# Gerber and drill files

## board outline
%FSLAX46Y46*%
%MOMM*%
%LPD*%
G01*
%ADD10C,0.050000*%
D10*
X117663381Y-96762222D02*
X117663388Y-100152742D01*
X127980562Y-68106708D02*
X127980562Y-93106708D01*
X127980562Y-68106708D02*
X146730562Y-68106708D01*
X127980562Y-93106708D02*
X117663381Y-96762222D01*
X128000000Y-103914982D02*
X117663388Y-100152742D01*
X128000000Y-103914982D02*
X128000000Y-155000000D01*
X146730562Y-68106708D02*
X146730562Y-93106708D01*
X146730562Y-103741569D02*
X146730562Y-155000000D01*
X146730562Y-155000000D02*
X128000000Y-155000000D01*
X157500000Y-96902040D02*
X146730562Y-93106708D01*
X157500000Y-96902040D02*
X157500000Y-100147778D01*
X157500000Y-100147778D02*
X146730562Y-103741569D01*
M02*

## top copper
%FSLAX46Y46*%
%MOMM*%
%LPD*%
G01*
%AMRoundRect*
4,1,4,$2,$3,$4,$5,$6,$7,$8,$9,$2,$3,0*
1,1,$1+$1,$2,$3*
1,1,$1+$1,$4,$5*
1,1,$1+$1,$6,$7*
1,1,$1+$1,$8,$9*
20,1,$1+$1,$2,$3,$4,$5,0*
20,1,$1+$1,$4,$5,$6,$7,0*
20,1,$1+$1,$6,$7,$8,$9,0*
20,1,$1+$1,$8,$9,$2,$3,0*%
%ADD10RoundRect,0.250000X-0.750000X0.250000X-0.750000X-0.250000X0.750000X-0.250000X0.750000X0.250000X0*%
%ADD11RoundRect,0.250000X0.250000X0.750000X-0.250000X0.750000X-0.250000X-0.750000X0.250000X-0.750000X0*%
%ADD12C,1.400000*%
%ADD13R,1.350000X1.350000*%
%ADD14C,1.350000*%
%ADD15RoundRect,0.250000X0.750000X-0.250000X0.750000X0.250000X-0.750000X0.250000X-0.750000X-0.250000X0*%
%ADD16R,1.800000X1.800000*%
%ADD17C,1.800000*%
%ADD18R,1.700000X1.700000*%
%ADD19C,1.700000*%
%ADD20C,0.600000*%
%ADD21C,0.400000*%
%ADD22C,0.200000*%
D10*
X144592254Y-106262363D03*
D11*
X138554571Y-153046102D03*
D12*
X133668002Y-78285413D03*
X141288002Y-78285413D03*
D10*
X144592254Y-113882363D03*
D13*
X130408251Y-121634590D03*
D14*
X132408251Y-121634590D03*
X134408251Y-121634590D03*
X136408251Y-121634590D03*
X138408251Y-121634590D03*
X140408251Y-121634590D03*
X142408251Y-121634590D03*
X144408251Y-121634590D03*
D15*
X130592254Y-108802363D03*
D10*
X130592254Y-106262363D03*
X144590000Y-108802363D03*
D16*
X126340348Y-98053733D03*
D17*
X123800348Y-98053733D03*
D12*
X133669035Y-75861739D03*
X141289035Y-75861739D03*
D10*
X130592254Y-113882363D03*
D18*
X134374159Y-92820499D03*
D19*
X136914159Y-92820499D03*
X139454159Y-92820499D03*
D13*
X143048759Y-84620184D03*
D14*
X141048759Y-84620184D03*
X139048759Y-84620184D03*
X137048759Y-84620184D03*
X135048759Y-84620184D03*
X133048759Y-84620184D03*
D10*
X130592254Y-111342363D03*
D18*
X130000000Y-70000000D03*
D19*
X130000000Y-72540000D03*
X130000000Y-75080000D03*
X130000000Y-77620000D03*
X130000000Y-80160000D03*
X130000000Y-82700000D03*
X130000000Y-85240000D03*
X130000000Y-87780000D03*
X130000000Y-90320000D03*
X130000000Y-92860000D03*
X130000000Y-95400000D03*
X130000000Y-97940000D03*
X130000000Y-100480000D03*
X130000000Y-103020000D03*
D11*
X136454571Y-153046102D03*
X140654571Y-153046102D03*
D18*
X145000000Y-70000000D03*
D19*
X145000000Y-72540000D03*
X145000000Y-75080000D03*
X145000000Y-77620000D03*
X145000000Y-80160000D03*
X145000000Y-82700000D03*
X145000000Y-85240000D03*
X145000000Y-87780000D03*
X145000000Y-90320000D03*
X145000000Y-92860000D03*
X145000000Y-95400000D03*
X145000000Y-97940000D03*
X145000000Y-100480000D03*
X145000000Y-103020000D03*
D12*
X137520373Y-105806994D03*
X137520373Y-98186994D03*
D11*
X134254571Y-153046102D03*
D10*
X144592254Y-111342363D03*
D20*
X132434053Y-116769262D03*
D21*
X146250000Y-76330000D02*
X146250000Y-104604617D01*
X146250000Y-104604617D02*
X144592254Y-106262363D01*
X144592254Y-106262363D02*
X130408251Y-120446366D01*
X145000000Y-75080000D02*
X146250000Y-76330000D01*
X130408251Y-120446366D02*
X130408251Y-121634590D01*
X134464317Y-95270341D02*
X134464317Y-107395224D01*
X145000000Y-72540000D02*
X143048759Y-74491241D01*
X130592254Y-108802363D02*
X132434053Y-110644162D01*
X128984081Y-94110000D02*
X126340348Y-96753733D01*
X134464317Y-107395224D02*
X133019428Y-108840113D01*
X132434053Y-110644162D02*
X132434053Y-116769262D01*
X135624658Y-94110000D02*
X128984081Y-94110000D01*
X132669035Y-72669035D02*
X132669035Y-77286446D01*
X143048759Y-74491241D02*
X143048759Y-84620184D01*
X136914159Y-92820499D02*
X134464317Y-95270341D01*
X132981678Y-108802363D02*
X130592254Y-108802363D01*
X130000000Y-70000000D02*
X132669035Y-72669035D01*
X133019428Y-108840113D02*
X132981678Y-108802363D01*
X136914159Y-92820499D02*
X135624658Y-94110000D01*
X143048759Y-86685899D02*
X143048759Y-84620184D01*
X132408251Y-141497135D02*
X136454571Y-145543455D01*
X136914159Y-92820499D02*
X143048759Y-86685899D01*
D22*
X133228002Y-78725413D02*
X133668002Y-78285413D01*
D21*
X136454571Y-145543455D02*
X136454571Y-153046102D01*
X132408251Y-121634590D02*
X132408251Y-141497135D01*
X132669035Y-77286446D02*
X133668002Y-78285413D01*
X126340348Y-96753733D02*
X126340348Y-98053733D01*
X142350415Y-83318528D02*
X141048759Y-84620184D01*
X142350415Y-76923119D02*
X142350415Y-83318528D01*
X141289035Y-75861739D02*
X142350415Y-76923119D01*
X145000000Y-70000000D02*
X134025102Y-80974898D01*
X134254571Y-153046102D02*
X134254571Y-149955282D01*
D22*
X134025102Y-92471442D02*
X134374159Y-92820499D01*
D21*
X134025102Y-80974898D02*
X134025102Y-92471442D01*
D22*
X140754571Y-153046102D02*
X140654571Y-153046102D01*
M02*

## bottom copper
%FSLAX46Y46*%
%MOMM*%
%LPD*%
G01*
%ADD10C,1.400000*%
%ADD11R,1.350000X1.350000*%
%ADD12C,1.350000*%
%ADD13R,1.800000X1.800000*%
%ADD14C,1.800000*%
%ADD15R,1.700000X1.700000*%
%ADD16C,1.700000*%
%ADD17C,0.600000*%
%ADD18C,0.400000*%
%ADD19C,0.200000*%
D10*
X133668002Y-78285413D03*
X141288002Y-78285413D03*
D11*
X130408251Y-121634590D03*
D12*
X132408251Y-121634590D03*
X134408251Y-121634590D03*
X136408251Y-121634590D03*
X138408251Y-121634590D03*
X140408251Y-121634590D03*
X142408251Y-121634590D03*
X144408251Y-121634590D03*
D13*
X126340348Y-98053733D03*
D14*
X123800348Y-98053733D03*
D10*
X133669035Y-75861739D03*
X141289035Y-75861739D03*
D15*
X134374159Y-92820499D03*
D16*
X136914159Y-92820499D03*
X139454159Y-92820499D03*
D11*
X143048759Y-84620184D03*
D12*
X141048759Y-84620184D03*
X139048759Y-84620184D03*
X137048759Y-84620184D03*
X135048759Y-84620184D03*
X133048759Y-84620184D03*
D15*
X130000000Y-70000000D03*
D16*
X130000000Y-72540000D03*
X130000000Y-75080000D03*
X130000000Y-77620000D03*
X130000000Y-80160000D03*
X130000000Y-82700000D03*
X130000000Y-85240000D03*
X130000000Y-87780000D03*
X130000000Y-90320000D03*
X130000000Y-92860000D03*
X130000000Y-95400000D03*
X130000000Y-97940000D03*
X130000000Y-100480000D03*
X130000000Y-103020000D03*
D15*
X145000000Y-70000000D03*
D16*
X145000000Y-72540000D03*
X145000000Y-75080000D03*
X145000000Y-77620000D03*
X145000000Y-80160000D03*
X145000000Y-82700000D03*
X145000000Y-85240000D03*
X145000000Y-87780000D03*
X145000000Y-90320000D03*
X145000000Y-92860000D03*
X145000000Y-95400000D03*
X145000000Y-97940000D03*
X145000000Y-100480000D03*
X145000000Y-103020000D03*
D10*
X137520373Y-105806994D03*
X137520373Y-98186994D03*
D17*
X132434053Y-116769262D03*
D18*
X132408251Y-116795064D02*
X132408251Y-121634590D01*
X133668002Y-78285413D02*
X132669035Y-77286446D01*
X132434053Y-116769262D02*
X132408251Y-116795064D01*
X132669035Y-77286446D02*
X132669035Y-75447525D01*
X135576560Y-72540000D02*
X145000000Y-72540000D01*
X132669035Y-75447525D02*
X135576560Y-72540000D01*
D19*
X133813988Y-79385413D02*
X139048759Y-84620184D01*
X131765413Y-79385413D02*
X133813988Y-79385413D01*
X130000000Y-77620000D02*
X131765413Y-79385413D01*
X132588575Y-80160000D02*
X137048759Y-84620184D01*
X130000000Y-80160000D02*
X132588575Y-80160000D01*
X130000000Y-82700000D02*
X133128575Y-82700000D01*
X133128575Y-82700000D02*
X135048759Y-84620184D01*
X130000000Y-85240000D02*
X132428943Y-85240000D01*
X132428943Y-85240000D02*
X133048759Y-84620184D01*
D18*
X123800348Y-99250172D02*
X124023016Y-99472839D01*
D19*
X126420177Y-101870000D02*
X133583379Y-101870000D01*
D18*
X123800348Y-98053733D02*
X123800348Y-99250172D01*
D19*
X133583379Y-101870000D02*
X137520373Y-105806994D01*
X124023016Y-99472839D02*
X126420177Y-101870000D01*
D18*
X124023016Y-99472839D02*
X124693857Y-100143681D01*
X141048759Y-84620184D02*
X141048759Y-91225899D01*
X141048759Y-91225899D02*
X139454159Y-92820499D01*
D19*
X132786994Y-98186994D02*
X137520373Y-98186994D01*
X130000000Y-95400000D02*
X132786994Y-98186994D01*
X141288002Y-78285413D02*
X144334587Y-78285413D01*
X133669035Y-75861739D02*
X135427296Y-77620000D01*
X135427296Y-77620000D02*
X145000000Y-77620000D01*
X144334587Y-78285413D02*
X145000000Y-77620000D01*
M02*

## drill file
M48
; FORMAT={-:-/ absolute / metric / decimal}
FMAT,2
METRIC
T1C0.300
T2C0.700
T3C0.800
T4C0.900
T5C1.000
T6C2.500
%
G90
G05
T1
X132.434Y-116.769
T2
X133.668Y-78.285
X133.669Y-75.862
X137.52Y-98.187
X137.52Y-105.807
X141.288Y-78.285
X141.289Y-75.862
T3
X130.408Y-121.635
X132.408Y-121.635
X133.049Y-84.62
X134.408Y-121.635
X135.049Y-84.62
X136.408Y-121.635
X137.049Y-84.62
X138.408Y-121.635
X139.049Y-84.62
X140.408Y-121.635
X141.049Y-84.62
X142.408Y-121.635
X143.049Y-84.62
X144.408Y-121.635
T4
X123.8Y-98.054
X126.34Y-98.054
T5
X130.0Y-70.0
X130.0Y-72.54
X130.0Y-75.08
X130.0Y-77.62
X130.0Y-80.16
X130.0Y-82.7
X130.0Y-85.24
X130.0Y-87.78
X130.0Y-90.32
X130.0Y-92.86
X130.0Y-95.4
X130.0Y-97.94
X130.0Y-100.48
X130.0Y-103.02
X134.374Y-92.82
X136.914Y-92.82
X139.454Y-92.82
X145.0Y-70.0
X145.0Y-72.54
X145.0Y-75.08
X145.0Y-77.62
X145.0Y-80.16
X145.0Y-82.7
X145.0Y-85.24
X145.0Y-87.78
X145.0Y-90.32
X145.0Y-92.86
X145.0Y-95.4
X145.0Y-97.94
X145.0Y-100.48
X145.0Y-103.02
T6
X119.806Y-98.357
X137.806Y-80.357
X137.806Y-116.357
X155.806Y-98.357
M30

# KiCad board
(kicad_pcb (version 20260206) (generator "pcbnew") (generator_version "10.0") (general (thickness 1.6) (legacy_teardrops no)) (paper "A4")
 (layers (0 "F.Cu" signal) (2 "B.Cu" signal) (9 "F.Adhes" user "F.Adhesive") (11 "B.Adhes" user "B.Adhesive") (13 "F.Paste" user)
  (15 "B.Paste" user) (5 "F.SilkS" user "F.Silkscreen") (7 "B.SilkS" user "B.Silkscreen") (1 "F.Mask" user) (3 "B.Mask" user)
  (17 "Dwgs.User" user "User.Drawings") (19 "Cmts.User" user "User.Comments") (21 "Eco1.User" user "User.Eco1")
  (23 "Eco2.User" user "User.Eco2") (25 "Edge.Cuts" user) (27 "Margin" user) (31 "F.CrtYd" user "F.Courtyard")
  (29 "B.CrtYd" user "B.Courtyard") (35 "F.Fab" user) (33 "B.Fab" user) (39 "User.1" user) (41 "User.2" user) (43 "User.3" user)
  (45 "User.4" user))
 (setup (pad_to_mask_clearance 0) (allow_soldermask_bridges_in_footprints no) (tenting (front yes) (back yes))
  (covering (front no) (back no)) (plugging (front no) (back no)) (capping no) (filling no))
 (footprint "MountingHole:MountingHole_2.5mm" (layer "F.Cu") (at 146.772986 83.971093)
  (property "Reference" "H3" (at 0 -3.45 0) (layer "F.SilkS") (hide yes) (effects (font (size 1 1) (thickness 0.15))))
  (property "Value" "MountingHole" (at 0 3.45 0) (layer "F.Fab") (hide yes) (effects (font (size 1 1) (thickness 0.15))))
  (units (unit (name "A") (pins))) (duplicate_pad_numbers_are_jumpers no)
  (pad "" np_thru_hole circle (at 9.033 14.386) (size 2.5 2.5) (drill 2.5) (layers "*.Cu" "*.Mask")))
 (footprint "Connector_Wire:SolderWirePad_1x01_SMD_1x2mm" (layer "F.Cu") (at 144.592254 106.262363 -90)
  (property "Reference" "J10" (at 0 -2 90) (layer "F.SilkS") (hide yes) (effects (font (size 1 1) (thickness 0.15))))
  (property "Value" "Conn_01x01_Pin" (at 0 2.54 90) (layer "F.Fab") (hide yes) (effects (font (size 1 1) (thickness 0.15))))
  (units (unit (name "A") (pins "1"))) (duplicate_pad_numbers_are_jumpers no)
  (pad "1" smd roundrect (at 0 0 270) (size 1 2) (layers "F.Cu" "F.Mask") (roundrect_rratio 0.25) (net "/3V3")))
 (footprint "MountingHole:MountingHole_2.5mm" (layer "F.Cu") (at 118.705986 81.757093)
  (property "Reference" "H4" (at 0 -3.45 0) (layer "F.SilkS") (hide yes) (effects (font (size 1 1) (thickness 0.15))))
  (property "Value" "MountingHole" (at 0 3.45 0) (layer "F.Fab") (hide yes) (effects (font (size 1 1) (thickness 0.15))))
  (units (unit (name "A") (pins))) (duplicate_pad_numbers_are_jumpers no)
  (pad "" np_thru_hole circle (at 1.1 16.6) (size 2.5 2.5) (drill 2.5) (layers "*.Cu" "*.Mask")))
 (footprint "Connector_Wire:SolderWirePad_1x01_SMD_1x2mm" (layer "F.Cu") (at 138.554571 153.046102 180)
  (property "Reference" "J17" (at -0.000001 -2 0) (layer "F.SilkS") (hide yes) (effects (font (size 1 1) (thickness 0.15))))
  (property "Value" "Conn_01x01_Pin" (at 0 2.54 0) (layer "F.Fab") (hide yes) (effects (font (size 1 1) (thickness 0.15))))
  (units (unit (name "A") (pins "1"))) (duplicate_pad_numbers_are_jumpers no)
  (pad "1" smd roundrect (at 0 0 180) (size 1 2) (layers "F.Cu" "F.Mask") (roundrect_rratio 0.25) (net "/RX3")))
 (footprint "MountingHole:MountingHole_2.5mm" (layer "F.Cu") (at 138.881986 97.502093)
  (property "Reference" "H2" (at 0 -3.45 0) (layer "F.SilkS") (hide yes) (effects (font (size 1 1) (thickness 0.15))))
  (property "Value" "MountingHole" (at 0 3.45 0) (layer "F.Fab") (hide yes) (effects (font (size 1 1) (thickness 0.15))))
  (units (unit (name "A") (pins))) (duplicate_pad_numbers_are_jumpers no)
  (pad "" np_thru_hole circle (at -1.076 18.855) (size 2.5 2.5) (drill 2.5) (layers "*.Cu" "*.Mask")))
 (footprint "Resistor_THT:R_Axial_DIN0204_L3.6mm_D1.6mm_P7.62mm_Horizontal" (layer "F.Cu") (at 133.668002 78.285413)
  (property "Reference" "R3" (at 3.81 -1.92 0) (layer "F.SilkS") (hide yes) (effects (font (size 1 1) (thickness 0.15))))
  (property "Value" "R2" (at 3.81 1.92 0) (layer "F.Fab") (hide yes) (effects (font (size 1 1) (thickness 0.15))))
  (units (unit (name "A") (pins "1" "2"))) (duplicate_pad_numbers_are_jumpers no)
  (pad "1" thru_hole circle (at 0 0) (size 1.4 1.4) (drill 0.7) (layers "*.Cu" "*.Mask") (remove_unused_layers no) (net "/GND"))
  (pad "2" thru_hole circle (at 7.62 0) (size 1.4 1.4) (drill 0.7) (layers "*.Cu" "*.Mask") (remove_unused_layers no) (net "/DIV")))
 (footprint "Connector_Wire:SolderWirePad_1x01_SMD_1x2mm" (layer "F.Cu") (at 144.592254 113.882363 -90)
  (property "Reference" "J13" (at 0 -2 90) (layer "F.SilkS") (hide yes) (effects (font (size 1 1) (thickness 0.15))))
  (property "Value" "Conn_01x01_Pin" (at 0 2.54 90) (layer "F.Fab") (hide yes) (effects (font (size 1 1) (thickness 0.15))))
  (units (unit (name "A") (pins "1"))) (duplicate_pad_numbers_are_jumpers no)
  (pad "1" smd roundrect (at 0 0 270) (size 1 2) (layers "F.Cu" "F.Mask") (roundrect_rratio 0.25) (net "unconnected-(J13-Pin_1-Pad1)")))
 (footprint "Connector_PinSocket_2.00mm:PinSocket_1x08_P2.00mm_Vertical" (layer "F.Cu") (at 130.408251 121.63459 90)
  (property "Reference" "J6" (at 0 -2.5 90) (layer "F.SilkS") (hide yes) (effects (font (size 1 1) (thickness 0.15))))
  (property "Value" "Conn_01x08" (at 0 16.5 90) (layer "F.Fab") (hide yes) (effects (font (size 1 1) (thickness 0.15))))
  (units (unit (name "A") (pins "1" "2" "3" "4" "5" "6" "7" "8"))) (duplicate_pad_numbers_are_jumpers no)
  (pad "1" thru_hole rect (at 0 0 90) (size 1.35 1.35) (drill 0.8) (layers "*.Cu" "*.Mask") (remove_unused_layers no) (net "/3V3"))
  (pad "2" thru_hole circle (at 0 2 90) (size 1.35 1.35) (drill 0.8) (layers "*.Cu" "*.Mask") (remove_unused_layers no) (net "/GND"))
  (pad "3" thru_hole circle (at 0 4 90) (size 1.35 1.35) (drill 0.8) (layers "*.Cu" "*.Mask") (remove_unused_layers no) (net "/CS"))
  (pad "4" thru_hole circle (at 0 6 90) (size 1.35 1.35) (drill 0.8) (layers "*.Cu" "*.Mask") (remove_unused_layers no) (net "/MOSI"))
  (pad "5" thru_hole circle (at 0 8 90) (size 1.35 1.35) (drill 0.8) (layers "*.Cu" "*.Mask") (remove_unused_layers no) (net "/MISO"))
  (pad "6" thru_hole circle (at 0 10 90) (size 1.35 1.35) (drill 0.8) (layers "*.Cu" "*.Mask") (remove_unused_layers no) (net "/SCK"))
  (pad "7" thru_hole circle (at 0 12 90) (size 1.35 1.35) (drill 0.8) (layers "*.Cu" "*.Mask") (remove_unused_layers no) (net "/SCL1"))
  (pad "8" thru_hole circle (at 0 14 90) (size 1.35 1.35) (drill 0.8) (layers "*.Cu" "*.Mask") (remove_unused_layers no) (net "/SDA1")))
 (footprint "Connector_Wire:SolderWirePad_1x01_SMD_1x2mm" (layer "F.Cu") (at 130.592254 108.802363 90)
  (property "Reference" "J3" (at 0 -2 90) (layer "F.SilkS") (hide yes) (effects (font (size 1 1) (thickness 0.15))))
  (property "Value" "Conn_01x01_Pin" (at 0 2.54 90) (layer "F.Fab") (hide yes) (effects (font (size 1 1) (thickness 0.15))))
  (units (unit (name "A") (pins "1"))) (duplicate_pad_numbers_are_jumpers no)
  (pad "1" smd roundrect (at 0 0 90) (size 1 2) (layers "F.Cu" "F.Mask") (roundrect_rratio 0.25) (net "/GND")))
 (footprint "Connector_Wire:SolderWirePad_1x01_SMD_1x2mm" (layer "F.Cu") (at 130.592254 106.262363 -90)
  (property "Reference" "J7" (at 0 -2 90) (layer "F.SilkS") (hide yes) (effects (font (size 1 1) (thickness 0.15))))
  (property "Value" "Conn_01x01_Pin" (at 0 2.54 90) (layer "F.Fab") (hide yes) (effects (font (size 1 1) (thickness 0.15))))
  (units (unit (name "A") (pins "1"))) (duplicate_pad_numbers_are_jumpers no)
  (pad "1" smd roundrect (at 0 0 270) (size 1 2) (layers "F.Cu" "F.Mask") (roundrect_rratio 0.25) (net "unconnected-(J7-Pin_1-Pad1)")))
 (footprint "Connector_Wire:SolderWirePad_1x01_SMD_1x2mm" (layer "F.Cu") (at 144.59 108.802363 -90)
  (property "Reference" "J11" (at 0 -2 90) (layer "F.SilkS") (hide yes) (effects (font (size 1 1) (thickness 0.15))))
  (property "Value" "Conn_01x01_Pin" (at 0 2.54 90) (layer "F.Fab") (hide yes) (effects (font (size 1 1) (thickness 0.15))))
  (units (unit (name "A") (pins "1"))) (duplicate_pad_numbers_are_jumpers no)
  (pad "1" smd roundrect (at 0 0 270) (size 1 2) (layers "F.Cu" "F.Mask") (roundrect_rratio 0.25) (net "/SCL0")))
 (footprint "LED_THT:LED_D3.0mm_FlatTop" (layer "F.Cu") (at 126.340348 98.053733 180)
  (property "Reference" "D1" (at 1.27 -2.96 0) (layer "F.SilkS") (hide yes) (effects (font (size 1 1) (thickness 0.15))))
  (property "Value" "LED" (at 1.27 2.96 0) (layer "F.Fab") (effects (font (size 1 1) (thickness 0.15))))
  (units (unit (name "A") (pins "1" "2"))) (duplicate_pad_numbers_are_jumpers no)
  (pad "1" thru_hole rect (at 0 0 180) (size 1.8 1.8) (drill 0.9) (layers "*.Cu" "*.Mask") (remove_unused_layers no) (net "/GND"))
  (pad "2" thru_hole circle (at 2.54 0 180) (size 1.8 1.8) (drill 0.9) (layers "*.Cu" "*.Mask") (remove_unused_layers no) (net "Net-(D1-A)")))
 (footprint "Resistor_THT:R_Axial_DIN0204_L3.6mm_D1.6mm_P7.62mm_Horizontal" (layer "F.Cu") (at 133.669035 75.861739)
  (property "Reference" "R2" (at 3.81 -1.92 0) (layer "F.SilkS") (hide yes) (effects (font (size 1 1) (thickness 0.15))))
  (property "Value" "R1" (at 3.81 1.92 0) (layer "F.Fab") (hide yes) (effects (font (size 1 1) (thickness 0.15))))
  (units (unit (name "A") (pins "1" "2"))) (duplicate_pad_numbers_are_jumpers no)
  (pad "1" thru_hole circle (at 0 0) (size 1.4 1.4) (drill 0.7) (layers "*.Cu" "*.Mask") (remove_unused_layers no) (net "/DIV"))
  (pad "2" thru_hole circle (at 7.62 0) (size 1.4 1.4) (drill 0.7) (layers "*.Cu" "*.Mask") (remove_unused_layers no) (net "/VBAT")))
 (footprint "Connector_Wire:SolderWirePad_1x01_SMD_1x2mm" (layer "F.Cu") (at 130.592254 113.882363 -90)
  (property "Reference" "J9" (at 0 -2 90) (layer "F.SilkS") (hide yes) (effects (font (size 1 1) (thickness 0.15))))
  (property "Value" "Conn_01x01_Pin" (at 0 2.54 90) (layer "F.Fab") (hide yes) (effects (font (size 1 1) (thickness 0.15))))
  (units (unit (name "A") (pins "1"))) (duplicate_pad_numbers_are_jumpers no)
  (pad "1" smd roundrect (at 0 0 270) (size 1 2) (layers "F.Cu" "F.Mask") (roundrect_rratio 0.25) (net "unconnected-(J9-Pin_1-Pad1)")))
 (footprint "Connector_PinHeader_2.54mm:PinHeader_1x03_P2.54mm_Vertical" (layer "F.Cu") (at 134.374159 92.820499 90)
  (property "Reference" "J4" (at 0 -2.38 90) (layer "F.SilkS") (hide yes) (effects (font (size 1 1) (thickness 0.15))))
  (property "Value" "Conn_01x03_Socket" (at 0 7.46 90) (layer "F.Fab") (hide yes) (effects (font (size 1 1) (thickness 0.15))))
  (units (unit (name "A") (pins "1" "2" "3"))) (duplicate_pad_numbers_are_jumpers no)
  (pad "1" thru_hole rect (at 0 0 90) (size 1.7 1.7) (drill 1) (layers "*.Cu" "*.Mask") (remove_unused_layers no) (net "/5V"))
  (pad "2" thru_hole circle (at 0 2.54 90) (size 1.7 1.7) (drill 1) (layers "*.Cu" "*.Mask") (remove_unused_layers no) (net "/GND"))
  (pad "3" thru_hole circle (at 0 5.08 90) (size 1.7 1.7) (drill 1) (layers "*.Cu" "*.Mask") (remove_unused_layers no) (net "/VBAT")))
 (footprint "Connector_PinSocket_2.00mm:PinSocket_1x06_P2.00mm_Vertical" (layer "F.Cu") (at 143.048759 84.620184 -90)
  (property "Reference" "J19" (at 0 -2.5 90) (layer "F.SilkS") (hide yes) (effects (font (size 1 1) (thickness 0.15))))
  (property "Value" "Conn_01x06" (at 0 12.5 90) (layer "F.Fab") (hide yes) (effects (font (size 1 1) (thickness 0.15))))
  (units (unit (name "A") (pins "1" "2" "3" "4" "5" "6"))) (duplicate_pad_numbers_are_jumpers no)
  (pad "1" thru_hole rect (at 0 0 270) (size 1.35 1.35) (drill 0.8) (layers "*.Cu" "*.Mask") (remove_unused_layers no) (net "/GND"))
  (pad "2" thru_hole circle (at 0 2 270) (size 1.35 1.35) (drill 0.8) (layers "*.Cu" "*.Mask") (remove_unused_layers no) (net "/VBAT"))
  (pad "3" thru_hole circle (at 0 4 270) (size 1.35 1.35) (drill 0.8) (layers "*.Cu" "*.Mask") (remove_unused_layers no) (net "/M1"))
  (pad "4" thru_hole circle (at 0 6 270) (size 1.35 1.35) (drill 0.8) (layers "*.Cu" "*.Mask") (remove_unused_layers no) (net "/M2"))
  (pad "5" thru_hole circle (at 0 8 270) (size 1.35 1.35) (drill 0.8) (layers "*.Cu" "*.Mask") (remove_unused_layers no) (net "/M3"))
  (pad "6" thru_hole circle (at 0 10 270) (size 1.35 1.35) (drill 0.8) (layers "*.Cu" "*.Mask") (remove_unused_layers no) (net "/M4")))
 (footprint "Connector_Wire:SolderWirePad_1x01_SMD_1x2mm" (layer "F.Cu") (at 130.592254 111.342363 -90)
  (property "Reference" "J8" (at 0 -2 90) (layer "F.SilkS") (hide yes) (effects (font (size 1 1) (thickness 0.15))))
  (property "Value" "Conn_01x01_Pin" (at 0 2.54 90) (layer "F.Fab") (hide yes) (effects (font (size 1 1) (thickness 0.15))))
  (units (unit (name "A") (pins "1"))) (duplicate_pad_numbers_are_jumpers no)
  (pad "1" smd roundrect (at 0 0 270) (size 1 2) (layers "F.Cu" "F.Mask") (roundrect_rratio 0.25) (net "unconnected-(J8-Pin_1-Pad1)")))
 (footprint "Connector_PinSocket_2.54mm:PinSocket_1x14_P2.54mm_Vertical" (layer "F.Cu") (at 130 70)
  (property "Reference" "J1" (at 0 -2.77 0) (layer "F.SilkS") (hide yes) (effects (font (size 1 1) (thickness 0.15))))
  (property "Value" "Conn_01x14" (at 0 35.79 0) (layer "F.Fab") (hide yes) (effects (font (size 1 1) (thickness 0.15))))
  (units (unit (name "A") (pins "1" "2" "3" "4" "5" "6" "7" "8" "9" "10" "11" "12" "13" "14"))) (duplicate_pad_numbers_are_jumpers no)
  (pad "1" thru_hole rect (at 0 0) (size 1.7 1.7) (drill 1) (layers "*.Cu" "*.Mask") (remove_unused_layers no) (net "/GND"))
  (pad "2" thru_hole circle (at 0 2.54) (size 1.7 1.7) (drill 1) (layers "*.Cu" "*.Mask") (remove_unused_layers no)
   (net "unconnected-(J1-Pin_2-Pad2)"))
  (pad "3" thru_hole circle (at 0 5.08) (size 1.7 1.7) (drill 1) (layers "*.Cu" "*.Mask") (remove_unused_layers no)
   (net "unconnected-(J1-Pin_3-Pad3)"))
  (pad "4" thru_hole circle (at 0 7.62) (size 1.7 1.7) (drill 1) (layers "*.Cu" "*.Mask") (remove_unused_layers no) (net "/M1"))
  (pad "5" thru_hole circle (at 0 10.16) (size 1.7 1.7) (drill 1) (layers "*.Cu" "*.Mask") (remove_unused_layers no) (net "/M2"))
  (pad "6" thru_hole circle (at 0 12.7) (size 1.7 1.7) (drill 1) (layers "*.Cu" "*.Mask") (remove_unused_layers no) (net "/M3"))
  (pad "7" thru_hole circle (at 0 15.24) (size 1.7 1.7) (drill 1) (layers "*.Cu" "*.Mask") (remove_unused_layers no) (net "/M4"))
  (pad "8" thru_hole circle (at 0 17.78) (size 1.7 1.7) (drill 1) (layers "*.Cu" "*.Mask") (remove_unused_layers no)
   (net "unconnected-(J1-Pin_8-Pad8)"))
  (pad "9" thru_hole circle (at 0 20.32) (size 1.7 1.7) (drill 1) (layers "*.Cu" "*.Mask") (remove_unused_layers no)
   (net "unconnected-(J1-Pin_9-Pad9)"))
  (pad "10" thru_hole circle (at 0 22.86) (size 1.7 1.7) (drill 1) (layers "*.Cu" "*.Mask") (remove_unused_layers no)
   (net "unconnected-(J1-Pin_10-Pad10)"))
  (pad "11" thru_hole circle (at 0 25.4) (size 1.7 1.7) (drill 1) (layers "*.Cu" "*.Mask") (remove_unused_layers no) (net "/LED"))
  (pad "12" thru_hole circle (at 0 27.94) (size 1.7 1.7) (drill 1) (layers "*.Cu" "*.Mask") (remove_unused_layers no) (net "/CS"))
  (pad "13" thru_hole circle (at 0 30.48) (size 1.7 1.7) (drill 1) (layers "*.Cu" "*.Mask") (remove_unused_layers no) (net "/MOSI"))
  (pad "14" thru_hole circle (at 0 33.02) (size 1.7 1.7) (drill 1) (layers "*.Cu" "*.Mask") (remove_unused_layers no) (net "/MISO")))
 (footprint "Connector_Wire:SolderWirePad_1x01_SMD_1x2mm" (layer "F.Cu") (at 136.454571 153.046102 180)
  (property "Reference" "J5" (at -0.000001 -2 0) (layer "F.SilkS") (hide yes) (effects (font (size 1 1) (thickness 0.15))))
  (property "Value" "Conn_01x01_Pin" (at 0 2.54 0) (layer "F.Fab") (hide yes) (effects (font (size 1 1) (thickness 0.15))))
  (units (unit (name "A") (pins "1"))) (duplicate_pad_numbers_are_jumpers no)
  (pad "1" smd roundrect (at 0 0 180) (size 1 2) (layers "F.Cu" "F.Mask") (roundrect_rratio 0.25) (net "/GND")))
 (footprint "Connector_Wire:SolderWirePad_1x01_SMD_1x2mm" (layer "F.Cu") (at 140.654571 153.046102 180)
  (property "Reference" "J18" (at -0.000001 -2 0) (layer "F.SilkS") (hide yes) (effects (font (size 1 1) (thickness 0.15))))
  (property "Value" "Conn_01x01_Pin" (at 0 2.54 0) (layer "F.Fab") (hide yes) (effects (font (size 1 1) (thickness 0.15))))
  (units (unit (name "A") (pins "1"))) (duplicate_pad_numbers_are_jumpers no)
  (pad "1" smd roundrect (at 0 0 180) (size 1 2) (layers "F.Cu" "F.Mask") (roundrect_rratio 0.25) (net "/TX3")))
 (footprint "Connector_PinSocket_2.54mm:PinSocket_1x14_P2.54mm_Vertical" (layer "F.Cu") (at 145 70)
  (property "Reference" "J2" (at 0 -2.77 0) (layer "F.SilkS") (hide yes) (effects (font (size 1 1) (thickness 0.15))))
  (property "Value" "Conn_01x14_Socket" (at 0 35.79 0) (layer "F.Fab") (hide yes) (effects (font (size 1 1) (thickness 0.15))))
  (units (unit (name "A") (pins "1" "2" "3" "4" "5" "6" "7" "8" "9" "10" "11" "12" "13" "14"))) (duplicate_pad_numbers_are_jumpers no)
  (pad "1" thru_hole rect (at 0 0) (size 1.7 1.7) (drill 1) (layers "*.Cu" "*.Mask") (remove_unused_layers no) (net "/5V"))
  (pad "2" thru_hole circle (at 0 2.54) (size 1.7 1.7) (drill 1) (layers "*.Cu" "*.Mask") (remove_unused_layers no) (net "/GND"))
  (pad "3" thru_hole circle (at 0 5.08) (size 1.7 1.7) (drill 1) (layers "*.Cu" "*.Mask") (remove_unused_layers no) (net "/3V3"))
  (pad "4" thru_hole circle (at 0 7.62) (size 1.7 1.7) (drill 1) (layers "*.Cu" "*.Mask") (remove_unused_layers no) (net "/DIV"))
  (pad "5" thru_hole circle (at 0 10.16) (size 1.7 1.7) (drill 1) (layers "*.Cu" "*.Mask") (remove_unused_layers no)
   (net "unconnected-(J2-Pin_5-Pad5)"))
  (pad "6" thru_hole circle (at 0 12.7) (size 1.7 1.7) (drill 1) (layers "*.Cu" "*.Mask") (remove_unused_layers no)
   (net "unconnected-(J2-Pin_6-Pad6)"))
  (pad "7" thru_hole circle (at 0 15.24) (size 1.7 1.7) (drill 1) (layers "*.Cu" "*.Mask") (remove_unused_layers no)
   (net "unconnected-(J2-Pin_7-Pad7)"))
  (pad "8" thru_hole circle (at 0 17.78) (size 1.7 1.7) (drill 1) (layers "*.Cu" "*.Mask") (remove_unused_layers no) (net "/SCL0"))
  (pad "9" thru_hole circle (at 0 20.32) (size 1.7 1.7) (drill 1) (layers "*.Cu" "*.Mask") (remove_unused_layers no) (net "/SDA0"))
  (pad "10" thru_hole circle (at 0 22.86) (size 1.7 1.7) (drill 1) (layers "*.Cu" "*.Mask") (remove_unused_layers no) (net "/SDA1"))
  (pad "11" thru_hole circle (at 0 25.4) (size 1.7 1.7) (drill 1) (layers "*.Cu" "*.Mask") (remove_unused_layers no) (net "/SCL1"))
  (pad "12" thru_hole circle (at 0 27.94) (size 1.7 1.7) (drill 1) (layers "*.Cu" "*.Mask") (remove_unused_layers no) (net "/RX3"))
  (pad "13" thru_hole circle (at 0 30.48) (size 1.7 1.7) (drill 1) (layers "*.Cu" "*.Mask") (remove_unused_layers no) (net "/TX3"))
  (pad "14" thru_hole circle (at 0 33.02) (size 1.7 1.7) (drill 1) (layers "*.Cu" "*.Mask") (remove_unused_layers no) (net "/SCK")))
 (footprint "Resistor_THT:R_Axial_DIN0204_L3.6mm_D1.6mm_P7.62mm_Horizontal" (layer "F.Cu") (at 137.520373 104.556994 90)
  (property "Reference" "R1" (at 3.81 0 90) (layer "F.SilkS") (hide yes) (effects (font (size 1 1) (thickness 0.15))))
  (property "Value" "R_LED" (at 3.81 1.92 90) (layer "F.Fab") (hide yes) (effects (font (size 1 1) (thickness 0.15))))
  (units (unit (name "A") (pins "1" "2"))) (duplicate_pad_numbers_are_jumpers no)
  (pad "1" thru_hole circle (at -1.25 0 90) (size 1.4 1.4) (drill 0.7) (layers "*.Cu" "*.Mask") (remove_unused_layers no) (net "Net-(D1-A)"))
  (pad "2" thru_hole circle (at 6.37 0 90) (size 1.4 1.4) (drill 0.7) (layers "*.Cu" "*.Mask") (remove_unused_layers no) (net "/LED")))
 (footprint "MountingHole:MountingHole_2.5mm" (layer "F.Cu") (at 135.660024 83.928054 -135)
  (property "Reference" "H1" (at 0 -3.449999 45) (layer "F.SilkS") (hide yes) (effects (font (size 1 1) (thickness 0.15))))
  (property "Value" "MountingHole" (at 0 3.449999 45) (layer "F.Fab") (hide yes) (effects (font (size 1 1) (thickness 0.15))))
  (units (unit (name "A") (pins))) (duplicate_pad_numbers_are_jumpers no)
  (pad "" np_thru_hole circle (at -4.042475 1.007626 225) (size 2.5 2.5) (drill 2.5) (layers "*.Cu" "*.Mask")))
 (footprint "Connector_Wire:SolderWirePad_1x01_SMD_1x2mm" (layer "F.Cu") (at 134.254571 153.046102 180)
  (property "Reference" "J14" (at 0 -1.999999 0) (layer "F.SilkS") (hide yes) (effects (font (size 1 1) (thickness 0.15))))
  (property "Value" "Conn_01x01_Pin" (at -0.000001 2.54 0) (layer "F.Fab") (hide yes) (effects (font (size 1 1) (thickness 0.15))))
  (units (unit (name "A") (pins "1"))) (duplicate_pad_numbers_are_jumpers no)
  (pad "1" smd roundrect (at 0 0 180) (size 1 2) (layers "F.Cu" "F.Mask") (roundrect_rratio 0.25) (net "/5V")))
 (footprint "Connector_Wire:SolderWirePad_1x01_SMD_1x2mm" (layer "F.Cu") (at 144.592254 111.342363 -90)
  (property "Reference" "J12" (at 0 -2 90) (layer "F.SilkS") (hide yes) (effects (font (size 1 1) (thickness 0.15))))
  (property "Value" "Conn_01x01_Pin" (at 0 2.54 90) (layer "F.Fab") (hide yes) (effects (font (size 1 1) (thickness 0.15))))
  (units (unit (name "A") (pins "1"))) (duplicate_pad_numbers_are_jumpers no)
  (pad "1" smd roundrect (at 0 0 270) (size 1 2) (layers "F.Cu" "F.Mask") (roundrect_rratio 0.25) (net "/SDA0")))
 (gr_line (start 117.663381 96.762222) (end 117.663388 100.152742) (stroke (width 0.05) (type solid)) (layer "Edge.Cuts"))
 (gr_line (start 127.980562 68.106708) (end 127.980562 93.106708) (stroke (width 0.05) (type solid)) (layer "Edge.Cuts"))
 (gr_line (start 127.980562 68.106708) (end 146.730562 68.106708) (stroke (width 0.05) (type solid)) (layer "Edge.Cuts"))
 (gr_line (start 127.980562 93.106708) (end 117.663381 96.762222) (stroke (width 0.05) (type solid)) (layer "Edge.Cuts"))
 (gr_line (start 128 103.914982) (end 117.663388 100.152742) (stroke (width 0.05) (type solid)) (layer "Edge.Cuts"))
 (gr_line (start 128 103.914982) (end 128 155) (stroke (width 0.05) (type solid)) (layer "Edge.Cuts"))
 (gr_line (start 146.730562 68.106708) (end 146.730562 93.106708) (stroke (width 0.05) (type solid)) (layer "Edge.Cuts"))
 (gr_line (start 146.730562 103.741569) (end 146.730562 155) (stroke (width 0.05) (type solid)) (layer "Edge.Cuts"))
 (gr_line (start 146.730562 155) (end 128 155) (stroke (width 0.05) (type solid)) (layer "Edge.Cuts"))
 (gr_line (start 157.5 96.90204) (end 146.730562 93.106708) (stroke (width 0.05) (type solid)) (layer "Edge.Cuts"))
 (gr_line (start 157.5 96.90204) (end 157.5 100.147778) (stroke (width 0.05) (type solid)) (layer "Edge.Cuts"))
 (gr_line (start 157.5 100.147778) (end 146.730562 103.741569) (stroke (width 0.05) (type solid)) (layer "Edge.Cuts"))
 (segment (start 146.25 76.33) (end 146.25 104.604617) (width 0.4) (layer "F.Cu") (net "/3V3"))
 (segment (start 146.25 104.604617) (end 144.592254 106.262363) (width 0.4) (layer "F.Cu") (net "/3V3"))
 (segment (start 144.592254 106.262363) (end 130.408251 120.446366) (width 0.4) (layer "F.Cu") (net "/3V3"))
 (segment (start 145 75.08) (end 146.25 76.33) (width 0.4) (layer "F.Cu") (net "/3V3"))
 (segment (start 130.408251 120.446366) (end 130.408251 121.63459) (width 0.4) (layer "F.Cu") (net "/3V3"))
 (segment (start 134.464317 95.270341) (end 134.464317 107.395224) (width 0.4) (layer "F.Cu") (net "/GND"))
 (segment (start 145 72.54) (end 143.048759 74.491241) (width 0.4) (layer "F.Cu") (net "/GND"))
 (segment (start 130.592254 108.802363) (end 132.434053 110.644162) (width 0.4) (layer "F.Cu") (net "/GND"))
 (segment (start 128.984081 94.11) (end 126.340348 96.753733) (width 0.4) (layer "F.Cu") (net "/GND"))
 (segment (start 134.464317 107.395224) (end 133.019428 108.840113) (width 0.4) (layer "F.Cu") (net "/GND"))
 (segment (start 132.434053 110.644162) (end 132.434053 116.769262) (width 0.4) (layer "F.Cu") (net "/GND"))
 (segment (start 135.624658 94.11) (end 128.984081 94.11) (width 0.4) (layer "F.Cu") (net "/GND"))
 (segment (start 132.669035 72.669035) (end 132.669035 77.286446) (width 0.4) (layer "F.Cu") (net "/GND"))
 (segment (start 143.048759 74.491241) (end 143.048759 84.620184) (width 0.4) (layer "F.Cu") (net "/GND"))
 (segment (start 136.914159 92.820499) (end 134.464317 95.270341) (width 0.4) (layer "F.Cu") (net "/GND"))
 (segment (start 132.981678 108.802363) (end 130.592254 108.802363) (width 0.4) (layer "F.Cu") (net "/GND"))
 (segment (start 130 70) (end 132.669035 72.669035) (width 0.4) (layer "F.Cu") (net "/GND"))
 (segment (start 133.019428 108.840113) (end 132.981678 108.802363) (width 0.4) (layer "F.Cu") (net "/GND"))
 (segment (start 136.914159 92.820499) (end 135.624658 94.11) (width 0.4) (layer "F.Cu") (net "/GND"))
 (segment (start 143.048759 86.685899) (end 143.048759 84.620184) (width 0.4) (layer "F.Cu") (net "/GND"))
 (segment (start 132.408251 141.497135) (end 136.454571 145.543455) (width 0.4) (layer "F.Cu") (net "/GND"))
 (segment (start 136.914159 92.820499) (end 143.048759 86.685899) (width 0.4) (layer "F.Cu") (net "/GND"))
 (segment (start 133.228002 78.725413) (end 133.668002 78.285413) (width 0.2) (layer "F.Cu") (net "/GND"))
 (segment (start 136.454571 145.543455) (end 136.454571 153.046102) (width 0.4) (layer "F.Cu") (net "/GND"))
 (segment (start 132.408251 121.63459) (end 132.408251 141.497135) (width 0.4) (layer "F.Cu") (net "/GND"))
 (segment (start 132.669035 77.286446) (end 133.668002 78.285413) (width 0.4) (layer "F.Cu") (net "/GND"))
 (segment (start 126.340348 96.753733) (end 126.340348 98.053733) (width 0.4) (layer "F.Cu") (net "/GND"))
 (via (at 132.434053 116.769262) (size 0.6) (drill 0.3) (layers "F.Cu" "B.Cu") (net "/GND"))
 (segment (start 132.408251 116.795064) (end 132.408251 121.63459) (width 0.4) (layer "B.Cu") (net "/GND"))
 (segment (start 133.668002 78.285413) (end 132.669035 77.286446) (width 0.4) (layer "B.Cu") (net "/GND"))
 (segment (start 132.434053 116.769262) (end 132.408251 116.795064) (width 0.4) (layer "B.Cu") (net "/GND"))
 (segment (start 132.669035 77.286446) (end 132.669035 75.447525) (width 0.4) (layer "B.Cu") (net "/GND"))
 (segment (start 135.57656 72.54) (end 145 72.54) (width 0.4) (layer "B.Cu") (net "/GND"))
 (segment (start 132.669035 75.447525) (end 135.57656 72.54) (width 0.4) (layer "B.Cu") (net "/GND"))
 (segment (start 133.813988 79.385413) (end 139.048759 84.620184) (width 0.2) (layer "B.Cu") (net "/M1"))
 (segment (start 131.765413 79.385413) (end 133.813988 79.385413) (width 0.2) (layer "B.Cu") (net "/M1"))
 (segment (start 130 77.62) (end 131.765413 79.385413) (width 0.2) (layer "B.Cu") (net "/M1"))
 (segment (start 132.588575 80.16) (end 137.048759 84.620184) (width 0.2) (layer "B.Cu") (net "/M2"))
 (segment (start 130 80.16) (end 132.588575 80.16) (width 0.2) (layer "B.Cu") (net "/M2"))
 (segment (start 130 82.7) (end 133.128575 82.7) (width 0.2) (layer "B.Cu") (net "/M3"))
 (segment (start 133.128575 82.7) (end 135.048759 84.620184) (width 0.2) (layer "B.Cu") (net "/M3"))
 (segment (start 130 85.24) (end 132.428943 85.24) (width 0.2) (layer "B.Cu") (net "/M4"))
 (segment (start 132.428943 85.24) (end 133.048759 84.620184) (width 0.2) (layer "B.Cu") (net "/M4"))
 (segment (start 123.800348 99.250172) (end 124.023016 99.472839) (width 0.4) (layer "B.Cu") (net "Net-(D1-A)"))
 (segment (start 126.420177 101.87) (end 133.583379 101.87) (width 0.2) (layer "B.Cu") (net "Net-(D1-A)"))
 (segment (start 123.800348 98.053733) (end 123.800348 99.250172) (width 0.4) (layer "B.Cu") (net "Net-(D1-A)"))
 (segment (start 133.583379 101.87) (end 137.520373 105.806994) (width 0.2) (layer "B.Cu") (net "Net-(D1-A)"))
 (segment (start 124.023016 99.472839) (end 126.420177 101.87) (width 0.2) (layer "B.Cu") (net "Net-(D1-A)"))
 (segment (start 124.023016 99.472839) (end 124.693857 100.143681) (width 0.4) (layer "B.Cu") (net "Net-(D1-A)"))
 (segment (start 142.350415 83.318528) (end 141.048759 84.620184) (width 0.4) (layer "F.Cu") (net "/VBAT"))
 (segment (start 142.350415 76.923119) (end 142.350415 83.318528) (width 0.4) (layer "F.Cu") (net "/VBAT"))
 (segment (start 141.289035 75.861739) (end 142.350415 76.923119) (width 0.4) (layer "F.Cu") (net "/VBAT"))
 (segment (start 141.048759 84.620184) (end 141.048759 91.225899) (width 0.4) (layer "B.Cu") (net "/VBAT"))
 (segment (start 141.048759 91.225899) (end 139.454159 92.820499) (width 0.4) (layer "B.Cu") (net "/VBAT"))
 (segment (start 145 70) (end 134.025102 80.974898) (width 0.4) (layer "F.Cu") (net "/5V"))
 (segment (start 134.254571 153.046102) (end 134.254571 149.955282) (width 0.4) (layer "F.Cu") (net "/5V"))
 (segment (start 134.025102 92.471442) (end 134.374159 92.820499) (width 0.2) (layer "F.Cu") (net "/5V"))
 (segment (start 134.025102 80.974898) (end 134.025102 92.471442) (width 0.4) (layer "F.Cu") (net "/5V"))
 (segment (start 132.786994 98.186994) (end 137.520373 98.186994) (width 0.2) (layer "B.Cu") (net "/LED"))
 (segment (start 130 95.4) (end 132.786994 98.186994) (width 0.2) (layer "B.Cu") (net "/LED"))
 (segment (start 140.754571 153.046102) (end 140.654571 153.046102) (width 0.2) (layer "F.Cu") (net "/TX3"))
 (segment (start 141.288002 78.285413) (end 144.334587 78.285413) (width 0.2) (layer "B.Cu") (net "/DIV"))
 (segment (start 133.669035 75.861739) (end 135.427296 77.62) (width 0.2) (layer "B.Cu") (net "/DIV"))
 (segment (start 135.427296 77.62) (end 145 77.62) (width 0.2) (layer "B.Cu") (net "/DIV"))
 (segment (start 144.334587 78.285413) (end 145 77.62) (width 0.2) (layer "B.Cu") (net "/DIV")))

